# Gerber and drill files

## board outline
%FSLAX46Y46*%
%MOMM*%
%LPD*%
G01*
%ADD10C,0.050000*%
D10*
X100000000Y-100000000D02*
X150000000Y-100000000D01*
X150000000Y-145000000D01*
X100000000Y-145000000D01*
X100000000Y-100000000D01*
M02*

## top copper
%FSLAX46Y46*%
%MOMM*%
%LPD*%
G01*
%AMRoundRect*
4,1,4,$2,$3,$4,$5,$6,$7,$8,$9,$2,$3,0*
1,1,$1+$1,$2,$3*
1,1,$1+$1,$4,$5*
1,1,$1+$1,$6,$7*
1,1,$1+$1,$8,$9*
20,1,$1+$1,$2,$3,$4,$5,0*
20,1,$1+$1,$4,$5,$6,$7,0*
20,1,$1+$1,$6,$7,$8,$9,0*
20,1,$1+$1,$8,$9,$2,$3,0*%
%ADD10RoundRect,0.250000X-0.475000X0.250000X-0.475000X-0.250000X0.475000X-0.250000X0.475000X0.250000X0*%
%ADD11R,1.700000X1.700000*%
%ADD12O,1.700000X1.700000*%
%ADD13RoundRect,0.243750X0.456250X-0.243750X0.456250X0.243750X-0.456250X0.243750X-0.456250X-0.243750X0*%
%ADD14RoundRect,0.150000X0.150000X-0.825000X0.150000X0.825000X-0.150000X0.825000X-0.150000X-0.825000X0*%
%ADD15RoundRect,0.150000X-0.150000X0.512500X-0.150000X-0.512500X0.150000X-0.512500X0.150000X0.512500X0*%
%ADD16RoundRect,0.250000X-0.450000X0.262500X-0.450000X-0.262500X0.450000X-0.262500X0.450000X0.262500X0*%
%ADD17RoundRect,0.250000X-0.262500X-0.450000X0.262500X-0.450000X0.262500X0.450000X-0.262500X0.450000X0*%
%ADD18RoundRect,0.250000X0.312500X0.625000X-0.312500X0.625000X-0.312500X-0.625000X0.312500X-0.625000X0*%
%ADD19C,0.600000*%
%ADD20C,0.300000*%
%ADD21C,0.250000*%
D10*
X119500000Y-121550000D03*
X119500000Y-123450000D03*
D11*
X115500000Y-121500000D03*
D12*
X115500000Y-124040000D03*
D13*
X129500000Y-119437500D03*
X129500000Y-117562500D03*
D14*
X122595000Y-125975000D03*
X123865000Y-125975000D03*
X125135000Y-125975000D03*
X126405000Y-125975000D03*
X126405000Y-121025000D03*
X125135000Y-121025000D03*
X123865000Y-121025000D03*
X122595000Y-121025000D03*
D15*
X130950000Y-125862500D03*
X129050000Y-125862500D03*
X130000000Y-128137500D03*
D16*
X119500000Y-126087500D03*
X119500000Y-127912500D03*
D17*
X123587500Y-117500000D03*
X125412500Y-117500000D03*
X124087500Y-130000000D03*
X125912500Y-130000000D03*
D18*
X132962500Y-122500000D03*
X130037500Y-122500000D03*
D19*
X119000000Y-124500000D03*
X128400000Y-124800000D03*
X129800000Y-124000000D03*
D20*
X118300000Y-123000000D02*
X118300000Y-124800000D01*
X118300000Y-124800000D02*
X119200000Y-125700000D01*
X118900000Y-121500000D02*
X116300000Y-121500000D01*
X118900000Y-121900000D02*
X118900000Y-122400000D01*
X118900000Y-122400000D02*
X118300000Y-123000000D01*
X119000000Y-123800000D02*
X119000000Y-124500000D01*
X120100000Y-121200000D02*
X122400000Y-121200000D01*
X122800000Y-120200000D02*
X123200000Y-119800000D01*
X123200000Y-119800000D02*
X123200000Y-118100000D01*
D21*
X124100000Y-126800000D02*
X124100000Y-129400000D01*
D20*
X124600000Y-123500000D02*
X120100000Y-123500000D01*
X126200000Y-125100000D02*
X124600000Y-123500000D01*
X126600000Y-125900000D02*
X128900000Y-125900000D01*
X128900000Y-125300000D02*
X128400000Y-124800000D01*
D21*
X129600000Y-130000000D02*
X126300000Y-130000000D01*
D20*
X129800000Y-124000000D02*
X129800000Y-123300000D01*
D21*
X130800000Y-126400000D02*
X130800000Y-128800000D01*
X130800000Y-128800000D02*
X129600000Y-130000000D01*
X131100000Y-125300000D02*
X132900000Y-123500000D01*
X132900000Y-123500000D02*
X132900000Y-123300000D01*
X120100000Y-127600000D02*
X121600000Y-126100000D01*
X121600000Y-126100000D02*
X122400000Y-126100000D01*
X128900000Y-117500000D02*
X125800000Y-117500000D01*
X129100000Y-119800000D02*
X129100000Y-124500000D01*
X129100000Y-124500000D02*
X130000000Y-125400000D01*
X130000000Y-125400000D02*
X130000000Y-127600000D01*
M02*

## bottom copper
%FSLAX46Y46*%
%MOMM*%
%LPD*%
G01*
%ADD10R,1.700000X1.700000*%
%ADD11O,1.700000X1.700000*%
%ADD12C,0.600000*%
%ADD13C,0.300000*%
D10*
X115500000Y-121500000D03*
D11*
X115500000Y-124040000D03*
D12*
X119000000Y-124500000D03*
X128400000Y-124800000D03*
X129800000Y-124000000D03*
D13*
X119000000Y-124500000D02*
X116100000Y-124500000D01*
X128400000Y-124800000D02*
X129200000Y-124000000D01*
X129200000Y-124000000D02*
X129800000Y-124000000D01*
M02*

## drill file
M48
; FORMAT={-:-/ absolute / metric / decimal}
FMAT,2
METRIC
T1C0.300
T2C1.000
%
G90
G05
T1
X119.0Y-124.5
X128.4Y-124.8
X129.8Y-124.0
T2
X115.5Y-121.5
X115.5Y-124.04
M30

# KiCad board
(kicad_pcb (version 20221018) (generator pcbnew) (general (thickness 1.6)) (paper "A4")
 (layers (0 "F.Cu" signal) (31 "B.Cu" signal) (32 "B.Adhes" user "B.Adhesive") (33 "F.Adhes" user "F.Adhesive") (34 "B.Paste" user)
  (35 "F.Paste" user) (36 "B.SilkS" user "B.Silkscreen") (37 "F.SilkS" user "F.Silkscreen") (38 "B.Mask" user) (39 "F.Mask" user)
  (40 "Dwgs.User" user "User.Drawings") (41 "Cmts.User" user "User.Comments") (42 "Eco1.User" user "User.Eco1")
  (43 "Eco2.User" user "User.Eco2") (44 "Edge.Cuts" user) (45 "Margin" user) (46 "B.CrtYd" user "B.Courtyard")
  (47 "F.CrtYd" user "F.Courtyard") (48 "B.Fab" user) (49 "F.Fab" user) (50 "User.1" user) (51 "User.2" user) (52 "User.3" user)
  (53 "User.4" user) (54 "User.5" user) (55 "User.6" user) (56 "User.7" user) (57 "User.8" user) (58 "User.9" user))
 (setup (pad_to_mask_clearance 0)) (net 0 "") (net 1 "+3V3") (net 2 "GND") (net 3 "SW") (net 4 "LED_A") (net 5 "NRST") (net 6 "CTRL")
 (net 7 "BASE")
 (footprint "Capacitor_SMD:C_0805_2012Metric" (layer "F.Cu") (at 119.5 122.5 -90)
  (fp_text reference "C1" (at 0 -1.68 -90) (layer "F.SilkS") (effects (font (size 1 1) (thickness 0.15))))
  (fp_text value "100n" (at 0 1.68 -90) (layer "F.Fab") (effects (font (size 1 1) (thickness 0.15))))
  (pad "1" smd roundrect (at -0.95 0 270) (size 1 1.45) (layers "F.Cu" "F.Paste" "F.Mask") (roundrect_rratio 0.25) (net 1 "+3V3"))
  (pad "2" smd roundrect (at 0.95 0 270) (size 1 1.45) (layers "F.Cu" "F.Paste" "F.Mask") (roundrect_rratio 0.25) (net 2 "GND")))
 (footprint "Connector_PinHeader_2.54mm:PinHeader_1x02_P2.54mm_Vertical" (layer "F.Cu") (at 115.5 121.5)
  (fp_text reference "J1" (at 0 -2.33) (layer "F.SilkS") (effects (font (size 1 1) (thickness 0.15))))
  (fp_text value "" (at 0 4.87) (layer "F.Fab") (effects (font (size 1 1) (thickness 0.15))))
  (pad "1" thru_hole rect (at 0 0) (size 1.7 1.7) (drill 1) (layers "*.Cu" "*.Mask") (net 1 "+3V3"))
  (pad "2" thru_hole oval (at 0 2.54) (size 1.7 1.7) (drill 1) (layers "*.Cu" "*.Mask") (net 2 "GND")))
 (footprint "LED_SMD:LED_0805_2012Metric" (layer "F.Cu") (at 129.5 118.5 90)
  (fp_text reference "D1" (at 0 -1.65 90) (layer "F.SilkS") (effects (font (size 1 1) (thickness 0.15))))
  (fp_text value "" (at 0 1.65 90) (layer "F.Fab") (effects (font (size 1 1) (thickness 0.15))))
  (pad "1" smd roundrect (at -0.9375 0 90) (size 0.975 1.4) (layers "F.Cu" "F.Paste" "F.Mask") (roundrect_rratio 0.25) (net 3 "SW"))
  (pad "2" smd roundrect (at 0.9375 0 90) (size 0.975 1.4) (layers "F.Cu" "F.Paste" "F.Mask") (roundrect_rratio 0.25) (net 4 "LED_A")))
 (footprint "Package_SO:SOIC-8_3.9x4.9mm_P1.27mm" (layer "F.Cu") (at 124.5 123.5 90)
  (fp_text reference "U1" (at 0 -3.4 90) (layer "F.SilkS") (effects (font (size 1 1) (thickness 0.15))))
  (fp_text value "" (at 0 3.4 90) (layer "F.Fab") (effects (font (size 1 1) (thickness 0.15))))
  (pad "1" smd roundrect (at -2.475 -1.905 90) (size 1.95 0.6) (layers "F.Cu" "F.Paste" "F.Mask") (roundrect_rratio 0.25) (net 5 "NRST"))
  (pad "2" smd roundrect (at -2.475 -0.635 90) (size 1.95 0.6) (layers "F.Cu" "F.Paste" "F.Mask") (roundrect_rratio 0.25) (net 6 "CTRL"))
  (pad "3" smd roundrect (at -2.475 0.635 90) (size 1.95 0.6) (layers "F.Cu" "F.Paste" "F.Mask") (roundrect_rratio 0.25))
  (pad "4" smd roundrect (at -2.475 1.905 90) (size 1.95 0.6) (layers "F.Cu" "F.Paste" "F.Mask") (roundrect_rratio 0.25) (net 2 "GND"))
  (pad "5" smd roundrect (at 2.475 1.905 90) (size 1.95 0.6) (layers "F.Cu" "F.Paste" "F.Mask") (roundrect_rratio 0.25))
  (pad "6" smd roundrect (at 2.475 0.635 90) (size 1.95 0.6) (layers "F.Cu" "F.Paste" "F.Mask") (roundrect_rratio 0.25))
  (pad "7" smd roundrect (at 2.475 -0.635 90) (size 1.95 0.6) (layers "F.Cu" "F.Paste" "F.Mask") (roundrect_rratio 0.25))
  (pad "8" smd roundrect (at 2.475 -1.905 90) (size 1.95 0.6) (layers "F.Cu" "F.Paste" "F.Mask") (roundrect_rratio 0.25) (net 1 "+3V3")))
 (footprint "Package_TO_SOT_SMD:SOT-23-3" (layer "F.Cu") (at 130 127 -90)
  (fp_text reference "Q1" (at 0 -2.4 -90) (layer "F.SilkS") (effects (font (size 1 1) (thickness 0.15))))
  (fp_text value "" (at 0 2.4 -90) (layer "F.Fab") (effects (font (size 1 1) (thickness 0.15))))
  (pad "1" smd roundrect (at -1.1375 -0.95 270) (size 1.325 0.6) (layers "F.Cu" "F.Paste" "F.Mask") (roundrect_rratio 0.25) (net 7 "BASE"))
  (pad "2" smd roundrect (at -1.1375 0.95 270) (size 1.325 0.6) (layers "F.Cu" "F.Paste" "F.Mask") (roundrect_rratio 0.25) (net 2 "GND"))
  (pad "3" smd roundrect (at 1.1375 0 270) (size 1.325 0.6) (layers "F.Cu" "F.Paste" "F.Mask") (roundrect_rratio 0.25) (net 3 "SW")))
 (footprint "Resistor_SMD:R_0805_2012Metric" (layer "F.Cu") (at 119.5 127 -90)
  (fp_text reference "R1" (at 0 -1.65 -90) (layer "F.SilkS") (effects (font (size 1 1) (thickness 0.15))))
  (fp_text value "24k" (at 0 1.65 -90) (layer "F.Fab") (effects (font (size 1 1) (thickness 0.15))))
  (pad "1" smd roundrect (at -0.9125 0 270) (size 1.025 1.4) (layers "F.Cu" "F.Paste" "F.Mask") (roundrect_rratio 0.243902) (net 1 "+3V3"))
  (pad "2" smd roundrect (at 0.9125 0 270) (size 1.025 1.4) (layers "F.Cu" "F.Paste" "F.Mask") (roundrect_rratio 0.243902) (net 5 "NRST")))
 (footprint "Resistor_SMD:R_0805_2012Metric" (layer "F.Cu") (at 124.5 117.5)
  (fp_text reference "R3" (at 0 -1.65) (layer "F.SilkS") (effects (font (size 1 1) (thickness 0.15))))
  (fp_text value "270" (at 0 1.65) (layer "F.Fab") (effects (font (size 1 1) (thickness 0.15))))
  (pad "1" smd roundrect (at -0.9125 0) (size 1.025 1.4) (layers "F.Cu" "F.Paste" "F.Mask") (roundrect_rratio 0.243902) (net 1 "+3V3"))
  (pad "2" smd roundrect (at 0.9125 0) (size 1.025 1.4) (layers "F.Cu" "F.Paste" "F.Mask") (roundrect_rratio 0.243902) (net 4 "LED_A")))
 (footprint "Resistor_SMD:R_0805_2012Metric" (layer "F.Cu") (at 125 130)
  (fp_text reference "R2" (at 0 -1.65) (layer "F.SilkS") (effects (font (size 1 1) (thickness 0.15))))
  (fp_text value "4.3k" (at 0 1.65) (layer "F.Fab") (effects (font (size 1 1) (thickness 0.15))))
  (pad "1" smd roundrect (at -0.9125 0) (size 1.025 1.4) (layers "F.Cu" "F.Paste" "F.Mask") (roundrect_rratio 0.243902) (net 6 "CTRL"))
  (pad "2" smd roundrect (at 0.9125 0) (size 1.025 1.4) (layers "F.Cu" "F.Paste" "F.Mask") (roundrect_rratio 0.243902) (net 7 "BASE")))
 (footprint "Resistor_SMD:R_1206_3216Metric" (layer "F.Cu") (at 131.5 122.5 180)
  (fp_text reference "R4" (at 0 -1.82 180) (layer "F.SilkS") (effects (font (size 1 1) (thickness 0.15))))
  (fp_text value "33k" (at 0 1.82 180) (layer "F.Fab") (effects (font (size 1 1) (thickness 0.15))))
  (pad "1" smd roundrect (at -1.4625 0 180) (size 1.125 1.75) (layers "F.Cu" "F.Paste" "F.Mask") (roundrect_rratio 0.222222) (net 7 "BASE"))
  (pad "2" smd roundrect (at 1.4625 0 180) (size 1.125 1.75) (layers "F.Cu" "F.Paste" "F.Mask") (roundrect_rratio 0.222222) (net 2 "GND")))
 (gr_rect (start 100 100) (end 150 145) (stroke (width 0.05) (type default)) (fill none) (layer "Edge.Cuts"))
 (segment (start 118.3 123) (end 118.3 124.8) (width 0.3) (layer "F.Cu") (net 1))
 (segment (start 118.3 124.8) (end 119.2 125.7) (width 0.3) (layer "F.Cu") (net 1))
 (segment (start 118.9 121.5) (end 116.3 121.5) (width 0.3) (layer "F.Cu") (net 1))
 (segment (start 118.9 121.9) (end 118.9 122.4) (width 0.3) (layer "F.Cu") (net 1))
 (segment (start 118.9 122.4) (end 118.3 123) (width 0.3) (layer "F.Cu") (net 1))
 (segment (start 119 123.8) (end 119 124.5) (width 0.3) (layer "F.Cu") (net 2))
 (segment (start 120.1 121.2) (end 122.4 121.2) (width 0.3) (layer "F.Cu") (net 1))
 (segment (start 122.8 120.2) (end 123.2 119.8) (width 0.3) (layer "F.Cu") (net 1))
 (segment (start 123.2 119.8) (end 123.2 118.1) (width 0.3) (layer "F.Cu") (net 1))
 (segment (start 124.1 126.8) (end 124.1 129.4) (width 0.25) (layer "F.Cu") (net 6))
 (segment (start 124.6 123.5) (end 120.1 123.5) (width 0.3) (layer "F.Cu") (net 2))
 (segment (start 126.2 125.1) (end 124.6 123.5) (width 0.3) (layer "F.Cu") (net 2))
 (segment (start 126.6 125.9) (end 128.9 125.9) (width 0.3) (layer "F.Cu") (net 2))
 (segment (start 128.9 125.3) (end 128.4 124.8) (width 0.3) (layer "F.Cu") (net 2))
 (segment (start 129.6 130) (end 126.3 130) (width 0.25) (layer "F.Cu") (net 7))
 (segment (start 129.8 124) (end 129.8 123.3) (width 0.3) (layer "F.Cu") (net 2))
 (segment (start 130.8 126.4) (end 130.8 128.8) (width 0.25) (layer "F.Cu") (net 7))
 (segment (start 130.8 128.8) (end 129.6 130) (width 0.25) (layer "F.Cu") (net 7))
 (segment (start 131.1 125.3) (end 132.9 123.5) (width 0.25) (layer "F.Cu") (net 7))
 (segment (start 132.9 123.5) (end 132.9 123.3) (width 0.25) (layer "F.Cu") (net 7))
 (via (at 119 124.5) (size 0.6) (drill 0.3) (layers "F.Cu" "B.Cu") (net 2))
 (via (at 128.4 124.8) (size 0.6) (drill 0.3) (layers "F.Cu" "B.Cu") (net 2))
 (via (at 129.8 124) (size 0.6) (drill 0.3) (layers "F.Cu" "B.Cu") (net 2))
 (segment (start 119 124.5) (end 116.1 124.5) (width 0.3) (layer "B.Cu") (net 2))
 (segment (start 120.1 127.6) (end 121.6 126.1) (width 0.25) (layer "F.Cu") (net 5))
 (segment (start 121.6 126.1) (end 122.4 126.1) (width 0.25) (layer "F.Cu") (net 5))
 (segment (start 128.4 124.8) (end 129.2 124) (width 0.3) (layer "B.Cu") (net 2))
 (segment (start 128.9 117.5) (end 125.8 117.5) (width 0.25) (layer "F.Cu") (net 4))
 (segment (start 129.1 119.8) (end 129.1 124.5) (width 0.25) (layer "F.Cu") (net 3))
 (segment (start 129.1 124.5) (end 130 125.4) (width 0.25) (layer "F.Cu") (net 3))
 (segment (start 129.2 124) (end 129.8 124) (width 0.3) (layer "B.Cu") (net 2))
 (segment (start 130 125.4) (end 130 127.6) (width 0.25) (layer "F.Cu") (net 3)))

